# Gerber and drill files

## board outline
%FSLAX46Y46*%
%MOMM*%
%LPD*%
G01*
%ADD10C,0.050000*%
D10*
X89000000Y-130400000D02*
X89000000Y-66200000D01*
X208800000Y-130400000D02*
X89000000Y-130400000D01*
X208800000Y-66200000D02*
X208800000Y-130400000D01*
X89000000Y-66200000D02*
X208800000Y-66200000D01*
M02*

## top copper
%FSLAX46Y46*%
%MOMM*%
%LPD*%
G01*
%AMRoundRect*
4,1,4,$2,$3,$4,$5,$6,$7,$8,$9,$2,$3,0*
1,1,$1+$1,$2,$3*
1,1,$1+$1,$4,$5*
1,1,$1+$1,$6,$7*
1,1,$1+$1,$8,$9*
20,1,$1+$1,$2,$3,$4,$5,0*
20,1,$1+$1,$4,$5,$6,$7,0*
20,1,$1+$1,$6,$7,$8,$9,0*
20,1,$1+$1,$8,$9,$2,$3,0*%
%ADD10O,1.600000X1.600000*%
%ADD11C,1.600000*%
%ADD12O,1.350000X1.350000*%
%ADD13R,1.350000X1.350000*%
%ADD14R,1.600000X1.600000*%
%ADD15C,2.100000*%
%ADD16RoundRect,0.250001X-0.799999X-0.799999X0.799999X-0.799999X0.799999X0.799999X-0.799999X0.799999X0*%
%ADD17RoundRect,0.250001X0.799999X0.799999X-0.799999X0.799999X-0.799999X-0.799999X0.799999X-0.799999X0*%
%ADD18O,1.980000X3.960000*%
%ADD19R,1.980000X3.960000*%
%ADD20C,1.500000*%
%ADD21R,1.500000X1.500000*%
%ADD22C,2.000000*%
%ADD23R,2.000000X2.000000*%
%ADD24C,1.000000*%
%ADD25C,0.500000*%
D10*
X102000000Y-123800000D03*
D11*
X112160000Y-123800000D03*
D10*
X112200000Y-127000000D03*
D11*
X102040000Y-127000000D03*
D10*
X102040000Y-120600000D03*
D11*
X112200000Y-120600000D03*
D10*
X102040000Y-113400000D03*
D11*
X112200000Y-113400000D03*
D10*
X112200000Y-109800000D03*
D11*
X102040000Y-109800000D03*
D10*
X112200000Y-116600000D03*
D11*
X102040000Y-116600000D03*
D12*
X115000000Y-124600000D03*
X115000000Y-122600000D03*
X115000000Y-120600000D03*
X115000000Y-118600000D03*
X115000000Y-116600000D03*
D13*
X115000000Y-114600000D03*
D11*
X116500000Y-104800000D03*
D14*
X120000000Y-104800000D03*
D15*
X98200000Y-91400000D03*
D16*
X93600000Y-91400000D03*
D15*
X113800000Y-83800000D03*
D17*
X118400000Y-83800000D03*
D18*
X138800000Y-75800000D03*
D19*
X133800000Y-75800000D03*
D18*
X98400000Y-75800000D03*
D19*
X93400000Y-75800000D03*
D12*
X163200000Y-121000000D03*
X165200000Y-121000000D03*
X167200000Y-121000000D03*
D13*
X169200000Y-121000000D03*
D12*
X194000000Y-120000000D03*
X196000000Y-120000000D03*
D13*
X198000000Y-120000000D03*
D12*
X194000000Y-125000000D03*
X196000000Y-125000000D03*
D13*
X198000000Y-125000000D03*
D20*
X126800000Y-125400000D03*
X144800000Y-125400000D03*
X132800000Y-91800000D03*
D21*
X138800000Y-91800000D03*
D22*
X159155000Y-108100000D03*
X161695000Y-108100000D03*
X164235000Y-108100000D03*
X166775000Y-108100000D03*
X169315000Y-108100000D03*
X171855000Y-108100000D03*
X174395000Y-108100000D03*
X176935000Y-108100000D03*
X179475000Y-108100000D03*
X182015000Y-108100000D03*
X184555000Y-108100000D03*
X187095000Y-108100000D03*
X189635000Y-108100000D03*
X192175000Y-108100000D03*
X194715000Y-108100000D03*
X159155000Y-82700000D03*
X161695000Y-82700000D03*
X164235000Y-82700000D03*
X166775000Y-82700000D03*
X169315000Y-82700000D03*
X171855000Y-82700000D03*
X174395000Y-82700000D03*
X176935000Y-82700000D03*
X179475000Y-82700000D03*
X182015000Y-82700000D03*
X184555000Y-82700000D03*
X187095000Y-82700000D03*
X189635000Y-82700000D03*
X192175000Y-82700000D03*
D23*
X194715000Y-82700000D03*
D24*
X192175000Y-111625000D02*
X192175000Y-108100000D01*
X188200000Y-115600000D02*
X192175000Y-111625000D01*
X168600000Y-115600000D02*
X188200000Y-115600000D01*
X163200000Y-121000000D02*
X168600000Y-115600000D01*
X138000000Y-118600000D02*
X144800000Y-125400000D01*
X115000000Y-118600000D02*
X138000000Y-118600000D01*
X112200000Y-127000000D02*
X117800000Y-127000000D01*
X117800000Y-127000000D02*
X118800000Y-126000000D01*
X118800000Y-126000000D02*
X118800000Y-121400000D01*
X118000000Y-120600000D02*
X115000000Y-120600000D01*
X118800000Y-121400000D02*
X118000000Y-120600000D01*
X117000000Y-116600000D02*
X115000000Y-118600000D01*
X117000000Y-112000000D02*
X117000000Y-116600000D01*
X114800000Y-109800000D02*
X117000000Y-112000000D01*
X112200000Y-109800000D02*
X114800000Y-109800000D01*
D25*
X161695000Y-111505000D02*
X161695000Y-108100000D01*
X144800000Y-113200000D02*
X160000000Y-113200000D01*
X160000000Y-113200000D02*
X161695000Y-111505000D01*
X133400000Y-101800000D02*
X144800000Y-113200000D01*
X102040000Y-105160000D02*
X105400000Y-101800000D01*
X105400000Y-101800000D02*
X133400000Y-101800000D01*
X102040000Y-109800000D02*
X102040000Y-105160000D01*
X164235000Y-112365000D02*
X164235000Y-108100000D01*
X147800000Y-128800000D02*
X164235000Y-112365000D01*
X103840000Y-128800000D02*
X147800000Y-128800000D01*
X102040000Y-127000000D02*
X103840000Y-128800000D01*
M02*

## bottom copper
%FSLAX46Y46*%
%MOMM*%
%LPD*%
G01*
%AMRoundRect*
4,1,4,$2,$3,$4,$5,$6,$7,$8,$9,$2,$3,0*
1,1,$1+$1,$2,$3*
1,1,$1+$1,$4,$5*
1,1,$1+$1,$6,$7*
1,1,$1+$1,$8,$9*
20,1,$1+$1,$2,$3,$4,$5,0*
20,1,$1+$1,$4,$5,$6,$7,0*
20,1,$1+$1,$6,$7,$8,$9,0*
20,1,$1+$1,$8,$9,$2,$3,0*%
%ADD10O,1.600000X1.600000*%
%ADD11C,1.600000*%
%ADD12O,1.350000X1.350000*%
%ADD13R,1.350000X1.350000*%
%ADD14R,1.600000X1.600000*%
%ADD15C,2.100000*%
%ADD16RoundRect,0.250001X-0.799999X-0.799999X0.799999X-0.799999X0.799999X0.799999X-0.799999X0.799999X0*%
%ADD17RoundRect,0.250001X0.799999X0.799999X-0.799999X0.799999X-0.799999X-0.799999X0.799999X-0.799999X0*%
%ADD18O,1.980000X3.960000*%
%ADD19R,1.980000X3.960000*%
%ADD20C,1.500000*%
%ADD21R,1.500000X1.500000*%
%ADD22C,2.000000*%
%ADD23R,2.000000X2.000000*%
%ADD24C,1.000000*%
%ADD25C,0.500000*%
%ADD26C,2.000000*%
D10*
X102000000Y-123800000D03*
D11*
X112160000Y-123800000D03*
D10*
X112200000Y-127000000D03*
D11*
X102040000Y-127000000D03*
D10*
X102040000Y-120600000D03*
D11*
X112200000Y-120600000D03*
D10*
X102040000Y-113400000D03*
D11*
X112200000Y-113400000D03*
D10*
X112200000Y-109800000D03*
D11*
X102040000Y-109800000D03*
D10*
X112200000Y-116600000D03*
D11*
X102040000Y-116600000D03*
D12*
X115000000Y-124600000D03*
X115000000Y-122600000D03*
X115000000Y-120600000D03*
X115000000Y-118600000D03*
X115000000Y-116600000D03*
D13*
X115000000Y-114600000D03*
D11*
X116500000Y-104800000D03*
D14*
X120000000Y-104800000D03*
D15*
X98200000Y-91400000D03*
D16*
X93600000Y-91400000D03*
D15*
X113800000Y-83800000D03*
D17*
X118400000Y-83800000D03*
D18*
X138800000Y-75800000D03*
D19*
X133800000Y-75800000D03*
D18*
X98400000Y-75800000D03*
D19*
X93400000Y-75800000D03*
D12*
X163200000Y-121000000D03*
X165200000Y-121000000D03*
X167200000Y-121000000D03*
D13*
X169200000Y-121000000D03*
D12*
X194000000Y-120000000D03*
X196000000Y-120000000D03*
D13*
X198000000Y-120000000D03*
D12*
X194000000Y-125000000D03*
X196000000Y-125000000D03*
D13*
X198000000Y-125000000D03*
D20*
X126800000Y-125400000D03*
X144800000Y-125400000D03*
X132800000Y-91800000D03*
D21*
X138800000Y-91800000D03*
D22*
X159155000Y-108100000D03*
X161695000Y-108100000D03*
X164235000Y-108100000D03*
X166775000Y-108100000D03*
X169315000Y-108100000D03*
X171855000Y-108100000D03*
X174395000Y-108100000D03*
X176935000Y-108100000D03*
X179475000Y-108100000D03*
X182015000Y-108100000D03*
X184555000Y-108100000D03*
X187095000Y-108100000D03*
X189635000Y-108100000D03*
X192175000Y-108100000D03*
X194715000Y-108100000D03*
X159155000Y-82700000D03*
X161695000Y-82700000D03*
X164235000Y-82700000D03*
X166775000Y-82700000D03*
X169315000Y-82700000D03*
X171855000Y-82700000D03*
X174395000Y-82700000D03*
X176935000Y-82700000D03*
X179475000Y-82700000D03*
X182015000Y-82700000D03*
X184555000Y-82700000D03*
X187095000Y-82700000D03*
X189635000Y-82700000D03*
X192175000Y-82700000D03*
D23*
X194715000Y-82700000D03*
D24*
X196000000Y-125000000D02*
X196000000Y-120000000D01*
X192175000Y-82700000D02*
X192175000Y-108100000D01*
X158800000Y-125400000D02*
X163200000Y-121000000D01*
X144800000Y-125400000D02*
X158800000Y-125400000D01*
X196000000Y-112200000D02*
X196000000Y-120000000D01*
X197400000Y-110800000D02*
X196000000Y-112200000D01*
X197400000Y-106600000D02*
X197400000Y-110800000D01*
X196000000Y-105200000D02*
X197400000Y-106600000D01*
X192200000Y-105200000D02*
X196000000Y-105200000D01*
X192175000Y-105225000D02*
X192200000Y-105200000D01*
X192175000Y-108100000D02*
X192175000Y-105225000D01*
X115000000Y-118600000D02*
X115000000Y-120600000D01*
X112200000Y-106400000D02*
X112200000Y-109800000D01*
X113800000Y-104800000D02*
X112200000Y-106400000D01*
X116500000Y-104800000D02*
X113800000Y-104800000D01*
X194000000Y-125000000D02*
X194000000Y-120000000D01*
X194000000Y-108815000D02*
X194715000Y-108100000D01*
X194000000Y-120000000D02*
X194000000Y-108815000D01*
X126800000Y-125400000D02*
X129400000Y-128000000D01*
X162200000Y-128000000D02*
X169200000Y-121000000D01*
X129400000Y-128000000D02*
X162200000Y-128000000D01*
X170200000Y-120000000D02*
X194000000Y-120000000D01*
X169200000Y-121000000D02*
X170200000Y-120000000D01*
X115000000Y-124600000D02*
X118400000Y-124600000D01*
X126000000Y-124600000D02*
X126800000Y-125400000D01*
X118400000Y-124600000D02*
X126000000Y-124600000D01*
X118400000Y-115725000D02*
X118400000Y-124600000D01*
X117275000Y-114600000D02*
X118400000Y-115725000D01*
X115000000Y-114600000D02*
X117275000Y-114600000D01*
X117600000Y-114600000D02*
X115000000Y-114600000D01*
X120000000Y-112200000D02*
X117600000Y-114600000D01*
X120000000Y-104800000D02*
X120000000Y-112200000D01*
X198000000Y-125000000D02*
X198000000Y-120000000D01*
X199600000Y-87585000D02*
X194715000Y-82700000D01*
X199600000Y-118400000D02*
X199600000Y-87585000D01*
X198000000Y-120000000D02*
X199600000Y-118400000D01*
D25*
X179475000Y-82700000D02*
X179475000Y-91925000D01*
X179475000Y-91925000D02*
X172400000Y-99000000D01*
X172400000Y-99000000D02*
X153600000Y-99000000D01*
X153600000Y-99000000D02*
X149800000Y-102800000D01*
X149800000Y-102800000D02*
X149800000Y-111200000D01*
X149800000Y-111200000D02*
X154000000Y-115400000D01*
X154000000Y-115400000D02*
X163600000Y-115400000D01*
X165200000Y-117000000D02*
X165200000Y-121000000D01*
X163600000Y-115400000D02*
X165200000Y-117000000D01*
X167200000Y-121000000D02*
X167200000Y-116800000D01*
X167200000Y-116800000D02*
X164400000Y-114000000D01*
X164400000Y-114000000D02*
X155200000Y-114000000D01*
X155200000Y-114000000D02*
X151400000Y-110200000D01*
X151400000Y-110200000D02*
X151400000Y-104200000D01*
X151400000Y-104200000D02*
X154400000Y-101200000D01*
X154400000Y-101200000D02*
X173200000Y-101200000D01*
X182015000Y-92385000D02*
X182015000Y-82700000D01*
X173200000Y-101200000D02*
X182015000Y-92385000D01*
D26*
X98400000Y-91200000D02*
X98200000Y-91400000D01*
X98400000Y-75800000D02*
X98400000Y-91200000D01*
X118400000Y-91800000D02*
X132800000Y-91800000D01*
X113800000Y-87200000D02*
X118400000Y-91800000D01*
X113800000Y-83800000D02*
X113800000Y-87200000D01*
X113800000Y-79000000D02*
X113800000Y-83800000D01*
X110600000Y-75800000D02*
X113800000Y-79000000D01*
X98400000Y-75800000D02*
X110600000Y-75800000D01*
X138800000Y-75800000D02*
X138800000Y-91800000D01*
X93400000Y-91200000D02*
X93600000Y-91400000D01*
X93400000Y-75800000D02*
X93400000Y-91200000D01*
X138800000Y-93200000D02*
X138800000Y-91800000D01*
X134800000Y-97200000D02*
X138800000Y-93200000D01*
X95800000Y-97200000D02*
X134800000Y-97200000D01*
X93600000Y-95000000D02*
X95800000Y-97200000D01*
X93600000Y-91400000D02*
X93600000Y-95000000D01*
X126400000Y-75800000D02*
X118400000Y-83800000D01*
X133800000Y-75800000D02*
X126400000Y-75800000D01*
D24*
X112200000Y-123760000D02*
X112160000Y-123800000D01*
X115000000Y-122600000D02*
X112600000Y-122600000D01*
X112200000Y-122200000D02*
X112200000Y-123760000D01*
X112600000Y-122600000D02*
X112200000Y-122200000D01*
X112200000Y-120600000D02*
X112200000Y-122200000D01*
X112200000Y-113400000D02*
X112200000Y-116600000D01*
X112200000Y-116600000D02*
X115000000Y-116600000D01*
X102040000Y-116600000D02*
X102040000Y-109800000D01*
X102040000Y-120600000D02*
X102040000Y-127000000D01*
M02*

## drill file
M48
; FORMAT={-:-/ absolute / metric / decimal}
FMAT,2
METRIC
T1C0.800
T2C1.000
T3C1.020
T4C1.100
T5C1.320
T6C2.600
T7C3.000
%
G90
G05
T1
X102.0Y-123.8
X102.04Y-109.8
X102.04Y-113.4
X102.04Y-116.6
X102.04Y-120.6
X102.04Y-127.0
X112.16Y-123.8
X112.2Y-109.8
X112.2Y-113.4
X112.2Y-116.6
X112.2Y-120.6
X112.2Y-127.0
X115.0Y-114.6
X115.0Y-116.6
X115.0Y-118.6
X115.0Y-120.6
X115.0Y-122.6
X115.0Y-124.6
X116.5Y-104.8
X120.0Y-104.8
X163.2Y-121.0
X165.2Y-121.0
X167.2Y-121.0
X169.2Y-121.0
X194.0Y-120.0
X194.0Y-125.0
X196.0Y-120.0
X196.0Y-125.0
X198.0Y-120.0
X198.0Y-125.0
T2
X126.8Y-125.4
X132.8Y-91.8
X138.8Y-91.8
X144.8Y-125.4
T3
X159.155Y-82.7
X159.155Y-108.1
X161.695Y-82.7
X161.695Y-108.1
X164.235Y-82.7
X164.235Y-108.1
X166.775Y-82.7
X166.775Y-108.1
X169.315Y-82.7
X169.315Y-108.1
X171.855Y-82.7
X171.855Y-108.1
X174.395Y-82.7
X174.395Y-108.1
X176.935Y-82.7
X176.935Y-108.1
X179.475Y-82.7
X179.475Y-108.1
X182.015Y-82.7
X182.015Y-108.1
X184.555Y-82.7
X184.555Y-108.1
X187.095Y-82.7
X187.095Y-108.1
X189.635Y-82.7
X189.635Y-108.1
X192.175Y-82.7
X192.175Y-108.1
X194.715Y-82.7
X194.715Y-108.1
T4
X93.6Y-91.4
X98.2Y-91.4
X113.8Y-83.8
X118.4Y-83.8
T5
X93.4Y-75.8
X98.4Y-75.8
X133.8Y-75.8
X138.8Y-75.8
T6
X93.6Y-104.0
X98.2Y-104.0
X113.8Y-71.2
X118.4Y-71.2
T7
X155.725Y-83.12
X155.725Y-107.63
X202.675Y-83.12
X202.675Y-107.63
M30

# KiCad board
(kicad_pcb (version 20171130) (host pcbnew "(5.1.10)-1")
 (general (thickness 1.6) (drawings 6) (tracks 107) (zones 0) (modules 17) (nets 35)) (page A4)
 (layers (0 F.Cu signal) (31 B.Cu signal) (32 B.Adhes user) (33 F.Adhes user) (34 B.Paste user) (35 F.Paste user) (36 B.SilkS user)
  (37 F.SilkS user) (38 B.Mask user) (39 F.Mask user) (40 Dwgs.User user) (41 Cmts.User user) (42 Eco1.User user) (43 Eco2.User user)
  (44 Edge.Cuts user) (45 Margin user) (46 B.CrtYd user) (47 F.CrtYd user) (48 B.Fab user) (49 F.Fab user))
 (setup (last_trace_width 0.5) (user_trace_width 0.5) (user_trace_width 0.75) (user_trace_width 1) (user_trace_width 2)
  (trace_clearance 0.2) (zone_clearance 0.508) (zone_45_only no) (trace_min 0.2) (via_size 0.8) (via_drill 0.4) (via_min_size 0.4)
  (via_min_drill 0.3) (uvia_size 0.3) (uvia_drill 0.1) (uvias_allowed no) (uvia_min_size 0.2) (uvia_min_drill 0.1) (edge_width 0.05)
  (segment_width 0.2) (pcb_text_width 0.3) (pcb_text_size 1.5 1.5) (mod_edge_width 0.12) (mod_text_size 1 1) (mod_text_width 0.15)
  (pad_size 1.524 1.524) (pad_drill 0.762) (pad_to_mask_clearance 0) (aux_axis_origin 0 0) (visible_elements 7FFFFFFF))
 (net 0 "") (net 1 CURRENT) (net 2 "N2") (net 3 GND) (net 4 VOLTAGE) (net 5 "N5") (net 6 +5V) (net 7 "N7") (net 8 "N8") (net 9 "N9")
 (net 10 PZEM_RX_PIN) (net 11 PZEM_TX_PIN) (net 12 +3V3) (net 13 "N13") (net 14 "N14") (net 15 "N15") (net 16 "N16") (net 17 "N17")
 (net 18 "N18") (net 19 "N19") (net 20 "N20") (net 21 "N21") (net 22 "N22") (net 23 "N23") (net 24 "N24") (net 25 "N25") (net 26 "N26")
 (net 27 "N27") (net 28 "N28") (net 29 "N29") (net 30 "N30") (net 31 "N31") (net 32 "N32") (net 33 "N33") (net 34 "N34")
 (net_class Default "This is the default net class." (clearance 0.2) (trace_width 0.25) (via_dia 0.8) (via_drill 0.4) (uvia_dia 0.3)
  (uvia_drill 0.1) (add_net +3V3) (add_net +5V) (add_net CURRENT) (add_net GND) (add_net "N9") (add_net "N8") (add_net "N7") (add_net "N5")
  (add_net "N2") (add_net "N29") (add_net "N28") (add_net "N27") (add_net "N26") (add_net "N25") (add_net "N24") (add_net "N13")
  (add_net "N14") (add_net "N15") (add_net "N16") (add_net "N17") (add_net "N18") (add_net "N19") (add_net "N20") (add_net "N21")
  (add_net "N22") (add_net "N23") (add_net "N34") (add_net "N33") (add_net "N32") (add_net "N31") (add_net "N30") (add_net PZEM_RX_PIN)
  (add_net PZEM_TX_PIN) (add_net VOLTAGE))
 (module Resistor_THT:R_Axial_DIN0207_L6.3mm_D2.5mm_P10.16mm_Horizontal (layer F.Cu) (at 112.16 123.8 180)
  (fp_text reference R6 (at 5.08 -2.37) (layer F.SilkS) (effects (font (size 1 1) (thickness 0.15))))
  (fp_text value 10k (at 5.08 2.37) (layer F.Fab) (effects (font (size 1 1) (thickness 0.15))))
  (pad 2 thru_hole oval (at 10.16 0 180) (size 1.6 1.6) (drill 0.8) (layers *.Cu *.Mask) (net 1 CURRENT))
  (pad 1 thru_hole circle (at 0 0 180) (size 1.6 1.6) (drill 0.8) (layers *.Cu *.Mask) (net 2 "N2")))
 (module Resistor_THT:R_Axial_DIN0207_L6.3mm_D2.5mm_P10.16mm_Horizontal (layer F.Cu) (at 102.04 127)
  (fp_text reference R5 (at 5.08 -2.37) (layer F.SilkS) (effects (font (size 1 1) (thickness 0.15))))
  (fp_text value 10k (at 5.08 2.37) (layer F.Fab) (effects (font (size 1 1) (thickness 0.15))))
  (pad 2 thru_hole oval (at 10.16 0) (size 1.6 1.6) (drill 0.8) (layers *.Cu *.Mask) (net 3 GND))
  (pad 1 thru_hole circle (at 0 0) (size 1.6 1.6) (drill 0.8) (layers *.Cu *.Mask) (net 1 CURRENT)))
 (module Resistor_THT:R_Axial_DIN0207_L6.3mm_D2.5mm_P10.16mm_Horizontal (layer F.Cu) (at 112.2 120.6 180)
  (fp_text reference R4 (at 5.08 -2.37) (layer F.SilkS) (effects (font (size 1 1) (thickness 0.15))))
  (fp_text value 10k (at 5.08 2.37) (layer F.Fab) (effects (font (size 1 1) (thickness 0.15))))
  (pad 2 thru_hole oval (at 10.16 0 180) (size 1.6 1.6) (drill 0.8) (layers *.Cu *.Mask) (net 1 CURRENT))
  (pad 1 thru_hole circle (at 0 0 180) (size 1.6 1.6) (drill 0.8) (layers *.Cu *.Mask) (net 2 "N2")))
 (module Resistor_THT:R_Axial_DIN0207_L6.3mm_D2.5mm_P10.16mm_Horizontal (layer F.Cu) (at 112.2 113.4 180)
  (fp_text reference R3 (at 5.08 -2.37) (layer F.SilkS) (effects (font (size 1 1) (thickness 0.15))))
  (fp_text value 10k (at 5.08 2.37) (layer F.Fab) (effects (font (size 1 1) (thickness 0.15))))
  (pad 2 thru_hole oval (at 10.16 0 180) (size 1.6 1.6) (drill 0.8) (layers *.Cu *.Mask) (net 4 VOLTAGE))
  (pad 1 thru_hole circle (at 0 0 180) (size 1.6 1.6) (drill 0.8) (layers *.Cu *.Mask) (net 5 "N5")))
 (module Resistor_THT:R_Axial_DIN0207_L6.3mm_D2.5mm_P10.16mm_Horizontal (layer F.Cu) (at 102.04 109.8)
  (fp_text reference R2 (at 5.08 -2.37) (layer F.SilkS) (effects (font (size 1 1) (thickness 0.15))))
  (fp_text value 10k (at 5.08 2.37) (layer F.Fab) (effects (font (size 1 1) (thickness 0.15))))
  (pad 2 thru_hole oval (at 10.16 0) (size 1.6 1.6) (drill 0.8) (layers *.Cu *.Mask) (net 3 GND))
  (pad 1 thru_hole circle (at 0 0) (size 1.6 1.6) (drill 0.8) (layers *.Cu *.Mask) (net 4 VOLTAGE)))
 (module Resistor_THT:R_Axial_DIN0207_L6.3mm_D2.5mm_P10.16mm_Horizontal (layer F.Cu) (at 102.04 116.6)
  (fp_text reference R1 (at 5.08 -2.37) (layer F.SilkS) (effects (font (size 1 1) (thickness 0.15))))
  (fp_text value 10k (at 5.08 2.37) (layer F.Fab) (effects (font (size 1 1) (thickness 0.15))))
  (pad 2 thru_hole oval (at 10.16 0) (size 1.6 1.6) (drill 0.8) (layers *.Cu *.Mask) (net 5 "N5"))
  (pad 1 thru_hole circle (at 0 0) (size 1.6 1.6) (drill 0.8) (layers *.Cu *.Mask) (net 4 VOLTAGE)))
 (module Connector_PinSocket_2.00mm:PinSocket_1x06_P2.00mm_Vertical (layer F.Cu) (at 115 114.6)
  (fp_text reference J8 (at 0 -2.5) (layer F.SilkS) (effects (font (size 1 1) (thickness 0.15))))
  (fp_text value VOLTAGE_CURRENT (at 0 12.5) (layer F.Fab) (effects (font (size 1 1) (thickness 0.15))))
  (pad 6 thru_hole oval (at 0 10) (size 1.35 1.35) (drill 0.8) (layers *.Cu *.Mask) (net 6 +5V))
  (pad 5 thru_hole oval (at 0 8) (size 1.35 1.35) (drill 0.8) (layers *.Cu *.Mask) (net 2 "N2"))
  (pad 4 thru_hole oval (at 0 6) (size 1.35 1.35) (drill 0.8) (layers *.Cu *.Mask) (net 3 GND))
  (pad 3 thru_hole oval (at 0 4) (size 1.35 1.35) (drill 0.8) (layers *.Cu *.Mask) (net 3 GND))
  (pad 2 thru_hole oval (at 0 2) (size 1.35 1.35) (drill 0.8) (layers *.Cu *.Mask) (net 5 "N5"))
  (pad 1 thru_hole rect (at 0 0) (size 1.35 1.35) (drill 0.8) (layers *.Cu *.Mask) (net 6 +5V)))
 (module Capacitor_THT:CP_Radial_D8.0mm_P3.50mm (layer F.Cu) (at 120 104.8 180)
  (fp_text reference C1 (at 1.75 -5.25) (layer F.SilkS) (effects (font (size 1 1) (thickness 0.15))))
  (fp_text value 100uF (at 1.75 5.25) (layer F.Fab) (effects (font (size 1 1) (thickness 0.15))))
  (pad 2 thru_hole circle (at 3.5 0 180) (size 1.6 1.6) (drill 0.8) (layers *.Cu *.Mask) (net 3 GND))
  (pad 1 thru_hole rect (at 0 0 180) (size 1.6 1.6) (drill 0.8) (layers *.Cu *.Mask) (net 6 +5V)))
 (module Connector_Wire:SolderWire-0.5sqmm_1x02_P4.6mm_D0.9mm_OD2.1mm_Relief (layer F.Cu) (at 93.6 91.4)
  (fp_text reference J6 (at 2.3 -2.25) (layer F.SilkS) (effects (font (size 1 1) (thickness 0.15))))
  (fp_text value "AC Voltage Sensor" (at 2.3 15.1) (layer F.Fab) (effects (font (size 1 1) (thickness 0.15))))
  (pad "" np_thru_hole circle (at 4.6 12.6) (size 2.6 2.6) (drill 2.6) (layers *.Cu *.Mask))
  (pad "" np_thru_hole circle (at 0 12.6) (size 2.6 2.6) (drill 2.6) (layers *.Cu *.Mask))
  (pad 2 thru_hole circle (at 4.6 0) (size 2.1 2.1) (drill 1.1) (layers *.Cu *.Mask) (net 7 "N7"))
  (pad 1 thru_hole roundrect (at 0 0) (size 2.1 2.1) (drill 1.1) (layers *.Cu *.Mask) (roundrect_rratio 0.119048) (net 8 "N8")))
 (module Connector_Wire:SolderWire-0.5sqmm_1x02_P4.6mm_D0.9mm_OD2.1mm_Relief (layer F.Cu) (at 118.4 83.8 180)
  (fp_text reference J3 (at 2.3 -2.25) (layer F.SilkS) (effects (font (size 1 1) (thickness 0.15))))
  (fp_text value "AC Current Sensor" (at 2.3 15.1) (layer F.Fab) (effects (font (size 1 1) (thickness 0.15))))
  (pad "" np_thru_hole circle (at 4.6 12.6 180) (size 2.6 2.6) (drill 2.6) (layers *.Cu *.Mask))
  (pad "" np_thru_hole circle (at 0 12.6 180) (size 2.6 2.6) (drill 2.6) (layers *.Cu *.Mask))
  (pad 2 thru_hole circle (at 4.6 0 180) (size 2.1 2.1) (drill 1.1) (layers *.Cu *.Mask) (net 7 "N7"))
  (pad 1 thru_hole roundrect (at 0 0 180) (size 2.1 2.1) (drill 1.1) (layers *.Cu *.Mask) (roundrect_rratio 0.119048) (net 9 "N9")))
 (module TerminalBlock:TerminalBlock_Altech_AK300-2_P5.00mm (layer F.Cu) (at 133.8 75.8)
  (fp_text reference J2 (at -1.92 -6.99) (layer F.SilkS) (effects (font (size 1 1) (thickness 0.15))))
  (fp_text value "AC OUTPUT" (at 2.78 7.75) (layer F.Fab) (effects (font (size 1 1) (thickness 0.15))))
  (pad 2 thru_hole oval (at 5 0) (size 1.98 3.96) (drill 1.32) (layers *.Cu *.Mask) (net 8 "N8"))
  (pad 1 thru_hole rect (at 0 0) (size 1.98 3.96) (drill 1.32) (layers *.Cu *.Mask) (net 9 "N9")))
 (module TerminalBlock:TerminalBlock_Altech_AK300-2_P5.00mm (layer F.Cu) (at 93.4 75.8)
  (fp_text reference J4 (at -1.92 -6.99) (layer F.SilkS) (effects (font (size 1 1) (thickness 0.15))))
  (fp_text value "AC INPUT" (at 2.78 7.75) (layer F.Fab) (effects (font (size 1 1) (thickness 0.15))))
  (pad 2 thru_hole oval (at 5 0) (size 1.98 3.96) (drill 1.32) (layers *.Cu *.Mask) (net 7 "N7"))
  (pad 1 thru_hole rect (at 0 0) (size 1.98 3.96) (drill 1.32) (layers *.Cu *.Mask) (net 8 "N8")))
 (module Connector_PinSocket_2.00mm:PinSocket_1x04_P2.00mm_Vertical (layer F.Cu) (at 169.2 121 270)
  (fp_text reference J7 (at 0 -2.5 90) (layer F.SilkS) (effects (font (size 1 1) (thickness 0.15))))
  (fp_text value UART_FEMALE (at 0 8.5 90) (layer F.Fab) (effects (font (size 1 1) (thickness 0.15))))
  (pad 4 thru_hole oval (at 0 6 270) (size 1.35 1.35) (drill 0.8) (layers *.Cu *.Mask) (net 3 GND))
  (pad 3 thru_hole oval (at 0 4 270) (size 1.35 1.35) (drill 0.8) (layers *.Cu *.Mask) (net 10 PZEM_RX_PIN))
  (pad 2 thru_hole oval (at 0 2 270) (size 1.35 1.35) (drill 0.8) (layers *.Cu *.Mask) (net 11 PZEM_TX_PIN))
  (pad 1 thru_hole rect (at 0 0 270) (size 1.35 1.35) (drill 0.8) (layers *.Cu *.Mask) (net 6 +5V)))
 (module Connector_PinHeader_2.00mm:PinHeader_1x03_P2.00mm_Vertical (layer F.Cu) (at 198 120 270)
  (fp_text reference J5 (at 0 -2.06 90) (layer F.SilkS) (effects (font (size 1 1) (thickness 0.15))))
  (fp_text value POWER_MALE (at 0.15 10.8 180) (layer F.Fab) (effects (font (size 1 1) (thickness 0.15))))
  (pad 3 thru_hole oval (at 0 4 270) (size 1.35 1.35) (drill 0.8) (layers *.Cu *.Mask) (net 6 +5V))
  (pad 2 thru_hole oval (at 0 2 270) (size 1.35 1.35) (drill 0.8) (layers *.Cu *.Mask) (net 3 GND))
  (pad 1 thru_hole rect (at 0 0 270) (size 1.35 1.35) (drill 0.8) (layers *.Cu *.Mask) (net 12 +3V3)))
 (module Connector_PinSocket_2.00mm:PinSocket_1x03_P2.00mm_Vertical (layer F.Cu) (at 198 125 270)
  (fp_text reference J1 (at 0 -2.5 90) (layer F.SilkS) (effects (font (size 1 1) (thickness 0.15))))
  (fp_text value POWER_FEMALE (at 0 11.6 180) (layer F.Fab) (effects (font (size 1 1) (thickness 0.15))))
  (pad 3 thru_hole oval (at 0 4 270) (size 1.35 1.35) (drill 0.8) (layers *.Cu *.Mask) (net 6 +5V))
  (pad 2 thru_hole oval (at 0 2 270) (size 1.35 1.35) (drill 0.8) (layers *.Cu *.Mask) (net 3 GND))
  (pad 1 thru_hole rect (at 0 0 270) (size 1.35 1.35) (drill 0.8) (layers *.Cu *.Mask) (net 12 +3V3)))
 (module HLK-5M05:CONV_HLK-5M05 (layer F.Cu) (at 135.8 108.6 270)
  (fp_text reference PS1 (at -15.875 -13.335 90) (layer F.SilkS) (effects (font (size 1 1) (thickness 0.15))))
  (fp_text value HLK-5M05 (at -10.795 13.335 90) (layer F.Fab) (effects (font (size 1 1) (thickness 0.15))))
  (pad 4 thru_hole circle (at 16.8 9 270) (size 1.5 1.5) (drill 1) (layers *.Cu *.Mask) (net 6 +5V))
  (pad 3 thru_hole circle (at 16.8 -9 270) (size 1.5 1.5) (drill 1) (layers *.Cu *.Mask) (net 3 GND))
  (pad 2 thru_hole circle (at -16.8 3 270) (size 1.5 1.5) (drill 1) (layers *.Cu *.Mask) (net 7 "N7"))
  (pad 1 thru_hole rect (at -16.8 -3 270) (size 1.5 1.5) (drill 1) (layers *.Cu *.Mask) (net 8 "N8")))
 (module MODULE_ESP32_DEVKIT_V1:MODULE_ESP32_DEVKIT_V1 (layer F.Cu) (at 179.2 95.4 270)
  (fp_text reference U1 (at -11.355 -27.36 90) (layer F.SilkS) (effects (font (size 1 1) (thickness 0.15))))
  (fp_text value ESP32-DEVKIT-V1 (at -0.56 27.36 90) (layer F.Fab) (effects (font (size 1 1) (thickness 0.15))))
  (pad None np_thru_hole circle (at -12.28 -23.475 270) (size 3 3) (drill 3) (layers *.Cu *.Mask))
  (pad None np_thru_hole circle (at 12.23 -23.475 270) (size 3 3) (drill 3) (layers *.Cu *.Mask))
  (pad None np_thru_hole circle (at 12.23 23.475 270) (size 3 3) (drill 3) (layers *.Cu *.Mask))
  (pad None np_thru_hole circle (at -12.28 23.475 270) (size 3 3) (drill 3) (layers *.Cu *.Mask))
  (pad 16 thru_hole circle (at 12.7 20.045 270) (size 2 2) (drill 1.02) (layers *.Cu *.Mask) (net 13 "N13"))
  (pad 17 thru_hole circle (at 12.7 17.505 270) (size 2 2) (drill 1.02) (layers *.Cu *.Mask) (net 4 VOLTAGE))
  (pad 18 thru_hole circle (at 12.7 14.965 270) (size 2 2) (drill 1.02) (layers *.Cu *.Mask) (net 1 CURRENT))
  (pad 19 thru_hole circle (at 12.7 12.425 270) (size 2 2) (drill 1.02) (layers *.Cu *.Mask) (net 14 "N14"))
  (pad 20 thru_hole circle (at 12.7 9.885 270) (size 2 2) (drill 1.02) (layers *.Cu *.Mask) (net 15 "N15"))
  (pad 21 thru_hole circle (at 12.7 7.345 270) (size 2 2) (drill 1.02) (layers *.Cu *.Mask) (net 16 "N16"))
  (pad 22 thru_hole circle (at 12.7 4.805 270) (size 2 2) (drill 1.02) (layers *.Cu *.Mask) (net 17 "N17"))
  (pad 23 thru_hole circle (at 12.7 2.265 270) (size 2 2) (drill 1.02) (layers *.Cu *.Mask) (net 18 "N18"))
  (pad 24 thru_hole circle (at 12.7 -0.275 270) (size 2 2) (drill 1.02) (layers *.Cu *.Mask) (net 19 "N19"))
  (pad 25 thru_hole circle (at 12.7 -2.815 270) (size 2 2) (drill 1.02) (layers *.Cu *.Mask) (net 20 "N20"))
  (pad 26 thru_hole circle (at 12.7 -5.355 270) (size 2 2) (drill 1.02) (layers *.Cu *.Mask) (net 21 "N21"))
  (pad 27 thru_hole circle (at 12.7 -7.895 270) (size 2 2) (drill 1.02) (layers *.Cu *.Mask) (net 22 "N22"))
  (pad 28 thru_hole circle (at 12.7 -10.435 270) (size 2 2) (drill 1.02) (layers *.Cu *.Mask) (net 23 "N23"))
  (pad 29 thru_hole circle (at 12.7 -12.975 270) (size 2 2) (drill 1.02) (layers *.Cu *.Mask) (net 3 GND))
  (pad 30 thru_hole circle (at 12.7 -15.515 270) (size 2 2) (drill 1.02) (layers *.Cu *.Mask) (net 6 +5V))
  (pad 15 thru_hole circle (at -12.7 20.045 270) (size 2 2) (drill 1.02) (layers *.Cu *.Mask) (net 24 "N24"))
  (pad 14 thru_hole circle (at -12.7 17.505 270) (size 2 2) (drill 1.02) (layers *.Cu *.Mask) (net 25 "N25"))
  (pad 13 thru_hole circle (at -12.7 14.965 270) (size 2 2) (drill 1.02) (layers *.Cu *.Mask) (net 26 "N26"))
  (pad 12 thru_hole circle (at -12.7 12.425 270) (size 2 2) (drill 1.02) (layers *.Cu *.Mask) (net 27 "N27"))
  (pad 11 thru_hole circle (at -12.7 9.885 270) (size 2 2) (drill 1.02) (layers *.Cu *.Mask) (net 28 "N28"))
  (pad 10 thru_hole circle (at -12.7 7.345 270) (size 2 2) (drill 1.02) (layers *.Cu *.Mask) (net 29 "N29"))
  (pad 9 thru_hole circle (at -12.7 4.805 270) (size 2 2) (drill 1.02) (layers *.Cu *.Mask) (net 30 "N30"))
  (pad 8 thru_hole circle (at -12.7 2.265 270) (size 2 2) (drill 1.02) (layers *.Cu *.Mask) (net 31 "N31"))
  (pad 7 thru_hole circle (at -12.7 -0.275 270) (size 2 2) (drill 1.02) (layers *.Cu *.Mask) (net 10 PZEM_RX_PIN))
  (pad 6 thru_hole circle (at -12.7 -2.815 270) (size 2 2) (drill 1.02) (layers *.Cu *.Mask) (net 11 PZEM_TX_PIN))
  (pad 5 thru_hole circle (at -12.7 -5.355 270) (size 2 2) (drill 1.02) (layers *.Cu *.Mask) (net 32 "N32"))
  (pad 4 thru_hole circle (at -12.7 -7.895 270) (size 2 2) (drill 1.02) (layers *.Cu *.Mask) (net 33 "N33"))
  (pad 3 thru_hole circle (at -12.7 -10.435 270) (size 2 2) (drill 1.02) (layers *.Cu *.Mask) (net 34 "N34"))
  (pad 2 thru_hole circle (at -12.7 -12.975 270) (size 2 2) (drill 1.02) (layers *.Cu *.Mask) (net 3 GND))
  (pad 1 thru_hole rect (at -12.7 -15.515 270) (size 2 2) (drill 1.02) (layers *.Cu *.Mask) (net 12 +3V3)))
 (gr_line (start 89 130.4) (end 89 66.2) (layer Edge.Cuts) (width 0.05))
 (gr_line (start 208.8 130.4) (end 89 130.4) (layer Edge.Cuts) (width 0.05))
 (gr_line (start 208.8 66.2) (end 208.8 130.4) (layer Edge.Cuts) (width 0.05))
 (gr_line (start 89 66.2) (end 208.8 66.2) (layer Edge.Cuts) (width 0.05))
 (segment (start 196 125) (end 196 120) (width 1) (layer B.Cu) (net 3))
 (segment (start 192.175 82.7) (end 192.175 108.1) (width 1) (layer B.Cu) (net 3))
 (segment (start 158.8 125.4) (end 163.2 121) (width 1) (layer B.Cu) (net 3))
 (segment (start 144.8 125.4) (end 158.8 125.4) (width 1) (layer B.Cu) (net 3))
 (segment (start 192.175 111.625) (end 192.175 108.1) (width 1) (layer F.Cu) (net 3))
 (segment (start 188.2 115.6) (end 192.175 111.625) (width 1) (layer F.Cu) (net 3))
 (segment (start 168.6 115.6) (end 188.2 115.6) (width 1) (layer F.Cu) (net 3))
 (segment (start 163.2 121) (end 168.6 115.6) (width 1) (layer F.Cu) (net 3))
 (segment (start 196 112.2) (end 196 120) (width 1) (layer B.Cu) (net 3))
 (segment (start 197.4 110.8) (end 196 112.2) (width 1) (layer B.Cu) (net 3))
 (segment (start 197.4 106.6) (end 197.4 110.8) (width 1) (layer B.Cu) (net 3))
 (segment (start 196 105.2) (end 197.4 106.6) (width 1) (layer B.Cu) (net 3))
 (segment (start 192.2 105.2) (end 196 105.2) (width 1) (layer B.Cu) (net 3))
 (segment (start 192.175 105.225) (end 192.2 105.2) (width 1) (layer B.Cu) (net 3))
 (segment (start 192.175 108.1) (end 192.175 105.225) (width 1) (layer B.Cu) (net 3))
 (segment (start 115 118.6) (end 115 120.6) (width 1) (layer B.Cu) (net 3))
 (segment (start 138 118.6) (end 144.8 125.4) (width 1) (layer F.Cu) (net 3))
 (segment (start 115 118.6) (end 138 118.6) (width 1) (layer F.Cu) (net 3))
 (segment (start 112.2 127) (end 117.8 127) (width 1) (layer F.Cu) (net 3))
 (segment (start 117.8 127) (end 118.8 126) (width 1) (layer F.Cu) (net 3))
 (segment (start 118.8 126) (end 118.8 121.4) (width 1) (layer F.Cu) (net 3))
 (segment (start 118 120.6) (end 115 120.6) (width 1) (layer F.Cu) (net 3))
 (segment (start 118.8 121.4) (end 118 120.6) (width 1) (layer F.Cu) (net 3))
 (segment (start 117 116.6) (end 115 118.6) (width 1) (layer F.Cu) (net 3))
 (segment (start 117 112) (end 117 116.6) (width 1) (layer F.Cu) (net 3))
 (segment (start 114.8 109.8) (end 117 112) (width 1) (layer F.Cu) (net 3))
 (segment (start 112.2 109.8) (end 114.8 109.8) (width 1) (layer F.Cu) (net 3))
 (segment (start 112.2 106.4) (end 112.2 109.8) (width 1) (layer B.Cu) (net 3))
 (segment (start 113.8 104.8) (end 112.2 106.4) (width 1) (layer B.Cu) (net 3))
 (segment (start 116.5 104.8) (end 113.8 104.8) (width 1) (layer B.Cu) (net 3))
 (segment (start 194 125) (end 194 120) (width 1) (layer B.Cu) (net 6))
 (segment (start 194 108.815) (end 194.715 108.1) (width 1) (layer B.Cu) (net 6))
 (segment (start 194 120) (end 194 108.815) (width 1) (layer B.Cu) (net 6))
 (segment (start 126.8 125.4) (end 129.4 128) (width 1) (layer B.Cu) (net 6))
 (segment (start 162.2 128) (end 169.2 121) (width 1) (layer B.Cu) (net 6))
 (segment (start 129.4 128) (end 162.2 128) (width 1) (layer B.Cu) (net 6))
 (segment (start 170.2 120) (end 194 120) (width 1) (layer B.Cu) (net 6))
 (segment (start 169.2 121) (end 170.2 120) (width 1) (layer B.Cu) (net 6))
 (segment (start 115 124.6) (end 118.4 124.6) (width 1) (layer B.Cu) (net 6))
 (segment (start 126 124.6) (end 126.8 125.4) (width 1) (layer B.Cu) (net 6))
 (segment (start 118.4 124.6) (end 126 124.6) (width 1) (layer B.Cu) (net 6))
 (segment (start 118.4 115.725) (end 118.4 124.6) (width 1) (layer B.Cu) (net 6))
 (segment (start 117.275 114.6) (end 118.4 115.725) (width 1) (layer B.Cu) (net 6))
 (segment (start 115 114.6) (end 117.275 114.6) (width 1) (layer B.Cu) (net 6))
 (segment (start 117.6 114.6) (end 115 114.6) (width 1) (layer B.Cu) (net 6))
 (segment (start 120 112.2) (end 117.6 114.6) (width 1) (layer B.Cu) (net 6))
 (segment (start 120 104.8) (end 120 112.2) (width 1) (layer B.Cu) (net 6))
 (segment (start 198 125) (end 198 120) (width 1) (layer B.Cu) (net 12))
 (segment (start 199.6 87.585) (end 194.715 82.7) (width 1) (layer B.Cu) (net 12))
 (segment (start 199.6 118.4) (end 199.6 87.585) (width 1) (layer B.Cu) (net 12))
 (segment (start 198 120) (end 199.6 118.4) (width 1) (layer B.Cu) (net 12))
 (segment (start 179.475 82.7) (end 179.475 91.925) (width 0.5) (layer B.Cu) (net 10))
 (segment (start 179.475 91.925) (end 172.4 99) (width 0.5) (layer B.Cu) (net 10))
 (segment (start 172.4 99) (end 153.6 99) (width 0.5) (layer B.Cu) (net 10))
 (segment (start 153.6 99) (end 149.8 102.8) (width 0.5) (layer B.Cu) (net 10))
 (segment (start 149.8 102.8) (end 149.8 111.2) (width 0.5) (layer B.Cu) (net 10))
 (segment (start 149.8 111.2) (end 154 115.4) (width 0.5) (layer B.Cu) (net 10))
 (segment (start 154 115.4) (end 163.6 115.4) (width 0.5) (layer B.Cu) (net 10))
 (segment (start 165.2 117) (end 165.2 121) (width 0.5) (layer B.Cu) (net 10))
 (segment (start 163.6 115.4) (end 165.2 117) (width 0.5) (layer B.Cu) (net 10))
 (segment (start 167.2 121) (end 167.2 116.8) (width 0.5) (layer B.Cu) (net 11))
 (segment (start 167.2 116.8) (end 164.4 114) (width 0.5) (layer B.Cu) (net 11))
 (segment (start 164.4 114) (end 155.2 114) (width 0.5) (layer B.Cu) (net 11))
 (segment (start 155.2 114) (end 151.4 110.2) (width 0.5) (layer B.Cu) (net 11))
 (segment (start 151.4 110.2) (end 151.4 104.2) (width 0.5) (layer B.Cu) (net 11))
 (segment (start 151.4 104.2) (end 154.4 101.2) (width 0.5) (layer B.Cu) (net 11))
 (segment (start 154.4 101.2) (end 173.2 101.2) (width 0.5) (layer B.Cu) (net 11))
 (segment (start 182.015 92.385) (end 182.015 82.7) (width 0.5) (layer B.Cu) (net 11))
 (segment (start 173.2 101.2) (end 182.015 92.385) (width 0.5) (layer B.Cu) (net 11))
 (segment (start 98.4 91.2) (end 98.2 91.4) (width 2) (layer B.Cu) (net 7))
 (segment (start 98.4 75.8) (end 98.4 91.2) (width 2) (layer B.Cu) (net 7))
 (segment (start 118.4 91.8) (end 132.8 91.8) (width 2) (layer B.Cu) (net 7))
 (segment (start 113.8 87.2) (end 118.4 91.8) (width 2) (layer B.Cu) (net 7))
 (segment (start 113.8 83.8) (end 113.8 87.2) (width 2) (layer B.Cu) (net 7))
 (segment (start 113.8 79) (end 113.8 83.8) (width 2) (layer B.Cu) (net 7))
 (segment (start 110.6 75.8) (end 113.8 79) (width 2) (layer B.Cu) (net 7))
 (segment (start 98.4 75.8) (end 110.6 75.8) (width 2) (layer B.Cu) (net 7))
 (segment (start 138.8 75.8) (end 138.8 91.8) (width 2) (layer B.Cu) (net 8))
 (segment (start 93.4 91.2) (end 93.6 91.4) (width 2) (layer B.Cu) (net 8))
 (segment (start 93.4 75.8) (end 93.4 91.2) (width 2) (layer B.Cu) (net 8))
 (segment (start 138.8 93.2) (end 138.8 91.8) (width 2) (layer B.Cu) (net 8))
 (segment (start 134.8 97.2) (end 138.8 93.2) (width 2) (layer B.Cu) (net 8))
 (segment (start 95.8 97.2) (end 134.8 97.2) (width 2) (layer B.Cu) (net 8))
 (segment (start 93.6 95) (end 95.8 97.2) (width 2) (layer B.Cu) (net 8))
 (segment (start 93.6 91.4) (end 93.6 95) (width 2) (layer B.Cu) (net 8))
 (segment (start 126.4 75.8) (end 118.4 83.8) (width 2) (layer B.Cu) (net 9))
 (segment (start 133.8 75.8) (end 126.4 75.8) (width 2) (layer B.Cu) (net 9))
 (segment (start 112.2 123.76) (end 112.16 123.8) (width 1) (layer B.Cu) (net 2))
 (segment (start 115 122.6) (end 112.6 122.6) (width 1) (layer B.Cu) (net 2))
 (segment (start 112.2 122.2) (end 112.2 123.76) (width 1) (layer B.Cu) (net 2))
 (segment (start 112.6 122.6) (end 112.2 122.2) (width 1) (layer B.Cu) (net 2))
 (segment (start 112.2 120.6) (end 112.2 122.2) (width 1) (layer B.Cu) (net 2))
 (segment (start 112.2 113.4) (end 112.2 116.6) (width 1) (layer B.Cu) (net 5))
 (segment (start 112.2 116.6) (end 115 116.6) (width 1) (layer B.Cu) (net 5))
 (segment (start 102.04 116.6) (end 102.04 109.8) (width 1) (layer B.Cu) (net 4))
 (segment (start 161.695 111.505) (end 161.695 108.1) (width 0.5) (layer F.Cu) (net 4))
 (segment (start 144.8 113.2) (end 160 113.2) (width 0.5) (layer F.Cu) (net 4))
 (segment (start 160 113.2) (end 161.695 111.505) (width 0.5) (layer F.Cu) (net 4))
 (segment (start 133.4 101.8) (end 144.8 113.2) (width 0.5) (layer F.Cu) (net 4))
 (segment (start 102.04 105.16) (end 105.4 101.8) (width 0.5) (layer F.Cu) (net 4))
 (segment (start 105.4 101.8) (end 133.4 101.8) (width 0.5) (layer F.Cu) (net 4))
 (segment (start 102.04 109.8) (end 102.04 105.16) (width 0.5) (layer F.Cu) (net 4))
 (segment (start 102.04 120.6) (end 102.04 127) (width 1) (layer B.Cu) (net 1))
 (segment (start 164.235 112.365) (end 164.235 108.1) (width 0.5) (layer F.Cu) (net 1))
 (segment (start 147.8 128.8) (end 164.235 112.365) (width 0.5) (layer F.Cu) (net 1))
 (segment (start 103.84 128.8) (end 147.8 128.8) (width 0.5) (layer F.Cu) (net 1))
 (segment (start 102.04 127) (end 103.84 128.8) (width 0.5) (layer F.Cu) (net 1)))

